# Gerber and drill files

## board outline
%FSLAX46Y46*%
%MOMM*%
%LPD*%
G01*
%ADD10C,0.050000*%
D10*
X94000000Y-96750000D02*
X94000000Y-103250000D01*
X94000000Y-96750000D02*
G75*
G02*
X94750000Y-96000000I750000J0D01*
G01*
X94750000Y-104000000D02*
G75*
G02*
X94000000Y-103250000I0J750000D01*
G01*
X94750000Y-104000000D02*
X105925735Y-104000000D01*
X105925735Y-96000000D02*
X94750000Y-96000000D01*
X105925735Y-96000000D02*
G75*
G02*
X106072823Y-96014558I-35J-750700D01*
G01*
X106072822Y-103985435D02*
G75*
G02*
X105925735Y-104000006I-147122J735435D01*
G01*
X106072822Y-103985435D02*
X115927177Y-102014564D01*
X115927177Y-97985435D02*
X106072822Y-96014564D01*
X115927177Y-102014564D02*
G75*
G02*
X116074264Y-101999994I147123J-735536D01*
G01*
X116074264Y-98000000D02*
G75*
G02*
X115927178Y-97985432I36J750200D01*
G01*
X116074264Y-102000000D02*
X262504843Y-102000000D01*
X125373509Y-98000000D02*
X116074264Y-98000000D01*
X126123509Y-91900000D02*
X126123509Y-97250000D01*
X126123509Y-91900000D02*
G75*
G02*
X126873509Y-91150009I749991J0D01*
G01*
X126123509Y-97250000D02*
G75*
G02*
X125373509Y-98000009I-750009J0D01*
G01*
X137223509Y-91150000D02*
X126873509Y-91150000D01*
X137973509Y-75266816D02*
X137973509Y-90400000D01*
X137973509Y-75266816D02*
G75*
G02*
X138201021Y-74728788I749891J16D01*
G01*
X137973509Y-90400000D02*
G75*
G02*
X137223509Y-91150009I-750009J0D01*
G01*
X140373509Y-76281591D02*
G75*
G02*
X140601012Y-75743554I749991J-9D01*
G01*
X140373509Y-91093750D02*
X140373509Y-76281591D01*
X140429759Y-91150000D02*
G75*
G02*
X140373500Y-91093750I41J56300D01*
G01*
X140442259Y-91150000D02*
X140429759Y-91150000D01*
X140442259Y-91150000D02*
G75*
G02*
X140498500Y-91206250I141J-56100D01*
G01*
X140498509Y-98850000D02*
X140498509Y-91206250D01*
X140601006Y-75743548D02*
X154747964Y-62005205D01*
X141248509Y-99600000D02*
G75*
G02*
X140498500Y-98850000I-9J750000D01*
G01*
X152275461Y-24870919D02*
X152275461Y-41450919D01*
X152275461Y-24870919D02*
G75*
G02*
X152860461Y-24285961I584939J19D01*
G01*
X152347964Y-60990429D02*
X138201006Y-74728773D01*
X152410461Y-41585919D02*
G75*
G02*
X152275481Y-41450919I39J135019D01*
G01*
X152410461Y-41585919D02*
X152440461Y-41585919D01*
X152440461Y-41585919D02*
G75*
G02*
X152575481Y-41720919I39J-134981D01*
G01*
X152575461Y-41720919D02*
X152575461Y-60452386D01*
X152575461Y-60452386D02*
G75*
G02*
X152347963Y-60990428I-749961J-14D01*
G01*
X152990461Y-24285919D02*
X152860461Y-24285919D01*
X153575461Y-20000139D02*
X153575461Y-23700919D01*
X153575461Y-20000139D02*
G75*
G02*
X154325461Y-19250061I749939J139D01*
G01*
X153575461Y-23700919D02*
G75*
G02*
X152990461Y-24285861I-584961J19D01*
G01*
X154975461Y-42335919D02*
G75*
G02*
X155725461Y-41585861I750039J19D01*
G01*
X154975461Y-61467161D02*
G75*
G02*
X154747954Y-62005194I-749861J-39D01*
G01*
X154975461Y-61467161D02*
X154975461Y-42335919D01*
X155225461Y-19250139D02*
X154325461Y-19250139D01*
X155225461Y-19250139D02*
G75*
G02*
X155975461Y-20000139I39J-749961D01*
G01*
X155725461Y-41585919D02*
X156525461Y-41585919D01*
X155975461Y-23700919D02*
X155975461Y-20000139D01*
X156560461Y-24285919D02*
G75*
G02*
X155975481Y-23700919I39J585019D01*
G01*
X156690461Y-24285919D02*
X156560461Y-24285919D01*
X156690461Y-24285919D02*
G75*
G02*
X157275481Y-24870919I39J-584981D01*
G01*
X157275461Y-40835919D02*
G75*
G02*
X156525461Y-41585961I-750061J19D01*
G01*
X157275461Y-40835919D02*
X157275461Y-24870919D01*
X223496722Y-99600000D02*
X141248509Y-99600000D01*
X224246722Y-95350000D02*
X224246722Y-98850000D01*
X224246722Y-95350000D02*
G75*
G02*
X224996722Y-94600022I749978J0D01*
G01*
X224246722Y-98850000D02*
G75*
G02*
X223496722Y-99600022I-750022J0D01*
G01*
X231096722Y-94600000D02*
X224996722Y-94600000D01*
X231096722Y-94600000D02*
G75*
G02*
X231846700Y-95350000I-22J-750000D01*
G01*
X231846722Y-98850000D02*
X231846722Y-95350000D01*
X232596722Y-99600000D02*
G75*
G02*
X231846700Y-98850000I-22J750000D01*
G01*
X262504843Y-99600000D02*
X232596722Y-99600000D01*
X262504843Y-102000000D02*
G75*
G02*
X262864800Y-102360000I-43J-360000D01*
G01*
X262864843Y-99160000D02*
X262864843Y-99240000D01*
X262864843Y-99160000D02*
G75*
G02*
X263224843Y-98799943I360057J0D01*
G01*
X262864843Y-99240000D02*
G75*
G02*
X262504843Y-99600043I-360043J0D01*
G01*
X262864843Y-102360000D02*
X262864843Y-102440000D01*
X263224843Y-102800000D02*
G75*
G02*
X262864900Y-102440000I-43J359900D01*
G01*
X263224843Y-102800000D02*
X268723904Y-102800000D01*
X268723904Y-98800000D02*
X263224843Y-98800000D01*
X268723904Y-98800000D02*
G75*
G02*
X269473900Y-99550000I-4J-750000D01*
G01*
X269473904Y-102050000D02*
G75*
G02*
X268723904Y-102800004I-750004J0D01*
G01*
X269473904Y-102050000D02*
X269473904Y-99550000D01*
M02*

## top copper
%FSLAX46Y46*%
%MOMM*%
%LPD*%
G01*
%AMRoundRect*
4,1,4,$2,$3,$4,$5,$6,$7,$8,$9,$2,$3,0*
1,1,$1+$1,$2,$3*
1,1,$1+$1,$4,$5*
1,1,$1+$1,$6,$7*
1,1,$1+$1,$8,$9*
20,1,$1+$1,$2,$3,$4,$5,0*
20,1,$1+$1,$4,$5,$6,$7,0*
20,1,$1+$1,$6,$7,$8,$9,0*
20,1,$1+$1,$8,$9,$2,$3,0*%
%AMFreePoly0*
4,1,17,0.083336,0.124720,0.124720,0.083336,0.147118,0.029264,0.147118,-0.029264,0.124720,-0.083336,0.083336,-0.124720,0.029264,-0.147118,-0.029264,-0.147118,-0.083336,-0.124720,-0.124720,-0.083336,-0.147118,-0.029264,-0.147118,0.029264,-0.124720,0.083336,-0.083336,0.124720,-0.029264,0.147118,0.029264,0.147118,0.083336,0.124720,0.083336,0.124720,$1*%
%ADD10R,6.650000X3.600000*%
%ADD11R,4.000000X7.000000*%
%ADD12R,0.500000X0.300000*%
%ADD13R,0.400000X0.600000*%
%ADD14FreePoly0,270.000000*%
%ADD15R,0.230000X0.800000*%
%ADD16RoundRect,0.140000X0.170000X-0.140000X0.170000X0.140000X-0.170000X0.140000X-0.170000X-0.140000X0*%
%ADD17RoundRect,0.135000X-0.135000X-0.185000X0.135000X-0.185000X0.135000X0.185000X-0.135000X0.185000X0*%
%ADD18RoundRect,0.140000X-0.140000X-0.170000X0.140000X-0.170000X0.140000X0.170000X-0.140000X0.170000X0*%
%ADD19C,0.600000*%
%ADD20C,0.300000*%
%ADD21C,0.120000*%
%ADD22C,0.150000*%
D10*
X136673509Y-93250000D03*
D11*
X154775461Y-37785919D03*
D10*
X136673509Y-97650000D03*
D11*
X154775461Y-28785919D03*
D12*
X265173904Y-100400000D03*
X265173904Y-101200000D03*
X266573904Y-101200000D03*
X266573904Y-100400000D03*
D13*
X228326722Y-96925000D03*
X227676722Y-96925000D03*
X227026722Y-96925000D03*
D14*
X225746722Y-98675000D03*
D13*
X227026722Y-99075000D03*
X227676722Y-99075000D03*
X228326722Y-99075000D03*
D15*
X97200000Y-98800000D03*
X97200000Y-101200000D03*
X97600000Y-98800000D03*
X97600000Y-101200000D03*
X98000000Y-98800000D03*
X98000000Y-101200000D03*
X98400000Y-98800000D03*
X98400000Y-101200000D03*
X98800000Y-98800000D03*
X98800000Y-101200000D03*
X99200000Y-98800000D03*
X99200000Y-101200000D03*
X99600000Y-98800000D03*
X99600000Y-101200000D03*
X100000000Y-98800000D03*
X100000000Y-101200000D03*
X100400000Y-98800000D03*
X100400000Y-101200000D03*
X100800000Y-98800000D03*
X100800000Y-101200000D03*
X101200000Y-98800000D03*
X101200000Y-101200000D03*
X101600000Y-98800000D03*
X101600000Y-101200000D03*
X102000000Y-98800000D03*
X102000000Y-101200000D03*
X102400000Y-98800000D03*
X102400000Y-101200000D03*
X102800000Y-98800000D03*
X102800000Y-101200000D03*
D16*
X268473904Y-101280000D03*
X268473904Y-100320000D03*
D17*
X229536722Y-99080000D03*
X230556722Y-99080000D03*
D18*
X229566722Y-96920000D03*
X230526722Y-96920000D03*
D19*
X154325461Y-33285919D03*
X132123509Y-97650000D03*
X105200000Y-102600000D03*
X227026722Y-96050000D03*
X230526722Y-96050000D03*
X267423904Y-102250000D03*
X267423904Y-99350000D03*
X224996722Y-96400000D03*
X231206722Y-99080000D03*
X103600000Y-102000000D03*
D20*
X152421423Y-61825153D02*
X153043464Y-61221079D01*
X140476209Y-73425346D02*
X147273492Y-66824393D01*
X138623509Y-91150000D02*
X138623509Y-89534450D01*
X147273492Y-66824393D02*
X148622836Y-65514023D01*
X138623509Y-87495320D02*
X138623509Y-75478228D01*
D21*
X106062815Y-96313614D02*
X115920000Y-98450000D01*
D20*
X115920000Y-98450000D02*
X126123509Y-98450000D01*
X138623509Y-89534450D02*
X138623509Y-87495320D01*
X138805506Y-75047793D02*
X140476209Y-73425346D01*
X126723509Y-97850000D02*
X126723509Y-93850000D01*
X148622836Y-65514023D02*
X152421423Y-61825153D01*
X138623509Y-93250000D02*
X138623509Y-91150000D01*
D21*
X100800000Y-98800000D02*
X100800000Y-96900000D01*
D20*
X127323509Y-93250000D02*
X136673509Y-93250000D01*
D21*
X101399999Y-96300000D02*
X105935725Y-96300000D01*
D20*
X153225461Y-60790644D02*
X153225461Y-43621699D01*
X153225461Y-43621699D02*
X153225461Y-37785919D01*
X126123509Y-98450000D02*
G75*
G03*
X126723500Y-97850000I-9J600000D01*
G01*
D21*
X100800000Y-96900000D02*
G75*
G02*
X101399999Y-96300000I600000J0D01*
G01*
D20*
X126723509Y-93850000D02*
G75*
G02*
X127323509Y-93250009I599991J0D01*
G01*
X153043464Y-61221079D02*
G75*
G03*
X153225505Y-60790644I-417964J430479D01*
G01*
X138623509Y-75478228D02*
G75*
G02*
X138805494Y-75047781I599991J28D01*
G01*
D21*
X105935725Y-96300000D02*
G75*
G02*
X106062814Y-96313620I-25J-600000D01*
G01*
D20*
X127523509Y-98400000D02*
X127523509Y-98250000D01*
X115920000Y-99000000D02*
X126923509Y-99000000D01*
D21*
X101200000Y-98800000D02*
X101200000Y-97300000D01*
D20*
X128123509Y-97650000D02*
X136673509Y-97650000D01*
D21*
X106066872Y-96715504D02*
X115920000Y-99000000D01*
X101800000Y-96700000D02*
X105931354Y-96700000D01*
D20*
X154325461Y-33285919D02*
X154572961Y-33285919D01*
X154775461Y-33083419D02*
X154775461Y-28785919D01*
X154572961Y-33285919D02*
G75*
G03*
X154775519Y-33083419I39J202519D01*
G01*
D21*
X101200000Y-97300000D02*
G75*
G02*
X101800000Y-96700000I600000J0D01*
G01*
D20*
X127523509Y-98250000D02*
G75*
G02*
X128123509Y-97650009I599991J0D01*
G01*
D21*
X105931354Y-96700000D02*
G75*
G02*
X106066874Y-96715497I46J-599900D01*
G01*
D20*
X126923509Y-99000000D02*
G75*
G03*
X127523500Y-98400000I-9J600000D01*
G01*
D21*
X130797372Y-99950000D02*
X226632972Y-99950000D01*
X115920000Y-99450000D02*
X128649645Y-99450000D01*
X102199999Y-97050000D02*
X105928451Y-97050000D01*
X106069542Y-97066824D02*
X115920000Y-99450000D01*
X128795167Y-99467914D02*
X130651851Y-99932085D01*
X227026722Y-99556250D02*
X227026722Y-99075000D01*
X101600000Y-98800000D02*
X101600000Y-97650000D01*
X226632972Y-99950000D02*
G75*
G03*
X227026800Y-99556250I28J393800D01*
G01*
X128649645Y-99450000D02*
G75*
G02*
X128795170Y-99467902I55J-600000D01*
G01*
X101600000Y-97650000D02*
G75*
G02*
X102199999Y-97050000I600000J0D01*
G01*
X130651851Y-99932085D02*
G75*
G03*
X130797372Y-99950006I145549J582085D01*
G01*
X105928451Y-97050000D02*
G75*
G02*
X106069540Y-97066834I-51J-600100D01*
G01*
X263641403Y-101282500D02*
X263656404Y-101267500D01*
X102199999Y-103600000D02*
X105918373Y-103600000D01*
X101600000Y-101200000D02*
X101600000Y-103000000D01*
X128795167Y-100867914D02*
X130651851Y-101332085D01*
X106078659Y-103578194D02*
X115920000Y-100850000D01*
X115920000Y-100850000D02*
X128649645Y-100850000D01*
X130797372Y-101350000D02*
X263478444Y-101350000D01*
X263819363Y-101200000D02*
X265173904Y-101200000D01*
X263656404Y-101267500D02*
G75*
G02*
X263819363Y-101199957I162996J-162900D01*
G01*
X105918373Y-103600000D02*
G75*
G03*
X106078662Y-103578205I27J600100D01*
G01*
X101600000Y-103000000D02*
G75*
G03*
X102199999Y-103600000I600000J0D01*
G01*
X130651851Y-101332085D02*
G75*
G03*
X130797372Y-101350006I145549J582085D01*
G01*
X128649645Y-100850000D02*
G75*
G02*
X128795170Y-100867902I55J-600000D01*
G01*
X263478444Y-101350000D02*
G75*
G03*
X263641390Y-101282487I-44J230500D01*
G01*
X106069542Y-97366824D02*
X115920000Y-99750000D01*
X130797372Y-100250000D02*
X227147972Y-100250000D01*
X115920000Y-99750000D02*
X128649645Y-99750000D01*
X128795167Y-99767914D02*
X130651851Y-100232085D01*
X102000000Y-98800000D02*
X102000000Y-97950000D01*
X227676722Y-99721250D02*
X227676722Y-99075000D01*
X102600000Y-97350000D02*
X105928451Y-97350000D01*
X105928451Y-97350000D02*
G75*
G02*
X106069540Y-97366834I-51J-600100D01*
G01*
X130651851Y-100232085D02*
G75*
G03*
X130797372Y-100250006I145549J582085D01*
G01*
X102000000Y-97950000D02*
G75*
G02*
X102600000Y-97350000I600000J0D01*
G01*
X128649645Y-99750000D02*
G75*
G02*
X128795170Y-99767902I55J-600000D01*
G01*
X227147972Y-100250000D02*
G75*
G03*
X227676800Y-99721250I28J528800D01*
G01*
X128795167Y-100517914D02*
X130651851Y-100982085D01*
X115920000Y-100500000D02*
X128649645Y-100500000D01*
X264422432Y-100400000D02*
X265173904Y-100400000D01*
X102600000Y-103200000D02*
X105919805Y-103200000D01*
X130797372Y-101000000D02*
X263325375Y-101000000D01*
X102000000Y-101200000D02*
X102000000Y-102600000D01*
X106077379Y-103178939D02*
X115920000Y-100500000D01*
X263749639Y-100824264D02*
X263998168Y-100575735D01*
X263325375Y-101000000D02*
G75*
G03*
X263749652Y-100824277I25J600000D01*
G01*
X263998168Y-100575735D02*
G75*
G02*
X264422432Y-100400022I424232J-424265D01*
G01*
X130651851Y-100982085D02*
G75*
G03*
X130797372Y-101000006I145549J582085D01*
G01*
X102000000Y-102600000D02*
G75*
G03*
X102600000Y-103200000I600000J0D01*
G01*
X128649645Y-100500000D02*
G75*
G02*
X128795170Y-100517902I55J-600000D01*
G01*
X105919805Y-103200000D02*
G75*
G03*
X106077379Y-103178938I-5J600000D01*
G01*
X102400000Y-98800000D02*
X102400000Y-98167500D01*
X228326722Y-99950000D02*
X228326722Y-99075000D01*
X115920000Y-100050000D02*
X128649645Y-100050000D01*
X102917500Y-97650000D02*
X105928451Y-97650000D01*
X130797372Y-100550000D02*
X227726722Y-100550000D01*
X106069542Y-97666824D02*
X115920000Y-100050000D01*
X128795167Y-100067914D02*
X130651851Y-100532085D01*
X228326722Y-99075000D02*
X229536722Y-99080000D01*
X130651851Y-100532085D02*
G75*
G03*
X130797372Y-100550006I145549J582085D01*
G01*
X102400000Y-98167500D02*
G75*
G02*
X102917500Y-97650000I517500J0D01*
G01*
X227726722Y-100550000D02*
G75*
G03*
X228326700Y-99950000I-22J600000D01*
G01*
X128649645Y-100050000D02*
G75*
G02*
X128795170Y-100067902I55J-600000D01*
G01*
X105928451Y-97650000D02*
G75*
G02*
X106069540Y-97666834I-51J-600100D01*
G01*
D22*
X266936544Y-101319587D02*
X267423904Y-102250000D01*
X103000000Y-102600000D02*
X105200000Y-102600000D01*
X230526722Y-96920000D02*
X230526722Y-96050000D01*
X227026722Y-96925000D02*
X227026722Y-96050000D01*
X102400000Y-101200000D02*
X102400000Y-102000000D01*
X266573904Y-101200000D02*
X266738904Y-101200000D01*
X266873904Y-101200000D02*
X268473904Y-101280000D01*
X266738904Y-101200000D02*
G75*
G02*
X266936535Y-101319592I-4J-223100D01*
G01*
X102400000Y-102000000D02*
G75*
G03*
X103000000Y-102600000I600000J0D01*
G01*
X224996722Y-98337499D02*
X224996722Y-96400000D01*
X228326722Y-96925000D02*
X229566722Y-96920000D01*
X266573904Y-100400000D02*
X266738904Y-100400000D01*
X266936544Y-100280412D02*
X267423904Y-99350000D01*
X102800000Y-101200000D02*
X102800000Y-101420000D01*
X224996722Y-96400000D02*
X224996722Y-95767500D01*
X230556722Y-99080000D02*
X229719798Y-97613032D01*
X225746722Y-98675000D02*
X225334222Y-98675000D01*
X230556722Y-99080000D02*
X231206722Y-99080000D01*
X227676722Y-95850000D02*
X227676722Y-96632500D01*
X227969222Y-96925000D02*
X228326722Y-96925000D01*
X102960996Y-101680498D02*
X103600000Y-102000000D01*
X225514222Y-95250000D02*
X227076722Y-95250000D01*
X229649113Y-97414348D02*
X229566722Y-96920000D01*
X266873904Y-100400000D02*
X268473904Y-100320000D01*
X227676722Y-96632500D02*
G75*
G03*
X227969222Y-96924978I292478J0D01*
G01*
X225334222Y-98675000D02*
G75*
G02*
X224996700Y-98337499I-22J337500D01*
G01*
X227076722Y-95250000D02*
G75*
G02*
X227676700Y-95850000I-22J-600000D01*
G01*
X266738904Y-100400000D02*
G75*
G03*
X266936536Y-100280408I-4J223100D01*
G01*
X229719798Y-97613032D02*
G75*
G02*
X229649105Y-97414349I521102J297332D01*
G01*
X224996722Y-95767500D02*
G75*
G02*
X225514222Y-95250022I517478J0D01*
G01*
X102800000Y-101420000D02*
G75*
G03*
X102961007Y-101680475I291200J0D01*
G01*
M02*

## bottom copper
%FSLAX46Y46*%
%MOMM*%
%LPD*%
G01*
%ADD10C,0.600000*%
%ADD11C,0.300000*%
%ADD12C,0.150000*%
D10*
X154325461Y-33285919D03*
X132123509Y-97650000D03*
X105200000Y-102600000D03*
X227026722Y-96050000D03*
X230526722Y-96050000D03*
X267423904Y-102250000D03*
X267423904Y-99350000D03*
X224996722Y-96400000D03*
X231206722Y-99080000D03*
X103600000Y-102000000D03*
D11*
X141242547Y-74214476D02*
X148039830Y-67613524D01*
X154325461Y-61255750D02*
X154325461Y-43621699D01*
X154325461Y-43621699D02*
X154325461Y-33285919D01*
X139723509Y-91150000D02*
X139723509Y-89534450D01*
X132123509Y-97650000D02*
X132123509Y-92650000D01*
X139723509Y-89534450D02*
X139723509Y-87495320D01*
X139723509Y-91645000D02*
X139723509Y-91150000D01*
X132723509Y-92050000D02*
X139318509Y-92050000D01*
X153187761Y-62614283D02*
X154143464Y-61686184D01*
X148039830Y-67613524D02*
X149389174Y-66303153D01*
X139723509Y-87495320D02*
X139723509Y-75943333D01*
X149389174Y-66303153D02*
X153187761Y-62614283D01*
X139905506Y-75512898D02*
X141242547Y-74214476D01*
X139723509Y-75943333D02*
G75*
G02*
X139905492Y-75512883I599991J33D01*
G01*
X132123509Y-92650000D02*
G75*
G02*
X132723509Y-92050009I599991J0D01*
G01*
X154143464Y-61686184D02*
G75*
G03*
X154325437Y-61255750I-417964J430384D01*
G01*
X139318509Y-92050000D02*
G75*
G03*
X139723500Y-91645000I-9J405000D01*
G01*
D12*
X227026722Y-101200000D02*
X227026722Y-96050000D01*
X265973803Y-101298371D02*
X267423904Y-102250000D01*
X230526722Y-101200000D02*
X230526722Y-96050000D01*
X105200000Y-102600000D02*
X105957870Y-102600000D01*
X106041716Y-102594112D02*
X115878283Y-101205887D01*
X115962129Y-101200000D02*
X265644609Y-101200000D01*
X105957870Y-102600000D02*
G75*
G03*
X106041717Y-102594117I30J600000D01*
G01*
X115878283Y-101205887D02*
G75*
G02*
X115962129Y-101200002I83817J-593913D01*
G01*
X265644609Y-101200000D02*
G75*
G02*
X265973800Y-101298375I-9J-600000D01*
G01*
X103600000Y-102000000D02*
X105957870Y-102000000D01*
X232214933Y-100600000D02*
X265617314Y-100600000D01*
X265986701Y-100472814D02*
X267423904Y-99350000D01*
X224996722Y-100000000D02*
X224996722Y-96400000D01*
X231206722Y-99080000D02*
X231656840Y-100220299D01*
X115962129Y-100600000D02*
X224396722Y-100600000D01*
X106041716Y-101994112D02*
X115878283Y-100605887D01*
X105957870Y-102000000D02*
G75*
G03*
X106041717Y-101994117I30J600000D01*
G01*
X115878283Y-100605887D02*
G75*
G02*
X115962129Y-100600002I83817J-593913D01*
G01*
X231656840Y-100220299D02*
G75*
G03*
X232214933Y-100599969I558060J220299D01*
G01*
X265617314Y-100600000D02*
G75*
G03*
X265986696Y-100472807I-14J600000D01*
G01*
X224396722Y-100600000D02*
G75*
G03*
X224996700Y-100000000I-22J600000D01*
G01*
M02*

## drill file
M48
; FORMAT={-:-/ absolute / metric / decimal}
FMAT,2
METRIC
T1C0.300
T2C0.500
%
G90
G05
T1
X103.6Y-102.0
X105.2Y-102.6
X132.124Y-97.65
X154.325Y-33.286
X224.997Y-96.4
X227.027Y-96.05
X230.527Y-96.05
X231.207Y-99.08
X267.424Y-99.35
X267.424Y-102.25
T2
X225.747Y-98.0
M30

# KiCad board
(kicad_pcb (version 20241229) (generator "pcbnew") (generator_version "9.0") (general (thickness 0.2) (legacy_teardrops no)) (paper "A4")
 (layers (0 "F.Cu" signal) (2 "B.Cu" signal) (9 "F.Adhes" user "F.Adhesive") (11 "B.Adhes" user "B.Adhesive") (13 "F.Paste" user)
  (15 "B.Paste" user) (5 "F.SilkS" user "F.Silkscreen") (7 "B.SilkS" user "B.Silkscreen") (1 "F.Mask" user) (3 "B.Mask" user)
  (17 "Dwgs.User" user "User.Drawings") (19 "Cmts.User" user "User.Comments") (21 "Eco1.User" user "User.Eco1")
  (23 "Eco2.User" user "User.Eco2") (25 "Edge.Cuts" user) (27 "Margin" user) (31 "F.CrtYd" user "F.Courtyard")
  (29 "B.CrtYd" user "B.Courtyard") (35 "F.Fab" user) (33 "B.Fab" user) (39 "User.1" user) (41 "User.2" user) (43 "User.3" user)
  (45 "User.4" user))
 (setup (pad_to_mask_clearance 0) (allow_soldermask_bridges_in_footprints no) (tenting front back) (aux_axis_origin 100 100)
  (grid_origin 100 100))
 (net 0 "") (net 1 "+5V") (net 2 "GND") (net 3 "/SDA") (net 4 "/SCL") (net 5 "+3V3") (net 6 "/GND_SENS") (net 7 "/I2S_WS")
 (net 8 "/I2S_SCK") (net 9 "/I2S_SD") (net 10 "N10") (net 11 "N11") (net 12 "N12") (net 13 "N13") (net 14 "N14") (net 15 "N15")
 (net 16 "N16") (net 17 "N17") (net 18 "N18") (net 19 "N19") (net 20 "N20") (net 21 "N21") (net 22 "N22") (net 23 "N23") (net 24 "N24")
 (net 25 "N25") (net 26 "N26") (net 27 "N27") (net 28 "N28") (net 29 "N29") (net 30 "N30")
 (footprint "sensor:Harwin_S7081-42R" (layer "F.Cu") (at 136.673509 93.25)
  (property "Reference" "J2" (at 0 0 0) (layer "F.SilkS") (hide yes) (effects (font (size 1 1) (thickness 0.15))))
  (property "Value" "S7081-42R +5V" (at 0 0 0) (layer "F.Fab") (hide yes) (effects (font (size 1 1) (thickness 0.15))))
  (pad "1" smd rect (at 0 0) (size 6.65 3.6) (layers "F.Cu" "F.Mask" "F.Paste") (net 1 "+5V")))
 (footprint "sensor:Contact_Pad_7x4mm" (layer "F.Cu") (at 154.775461 37.785919 90)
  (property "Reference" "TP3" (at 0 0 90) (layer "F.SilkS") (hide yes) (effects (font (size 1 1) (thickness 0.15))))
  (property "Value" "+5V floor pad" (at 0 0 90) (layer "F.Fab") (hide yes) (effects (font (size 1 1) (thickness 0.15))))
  (pad "1" smd rect (at 0 0 90) (size 7 4) (layers "F.Cu" "F.Mask") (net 1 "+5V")))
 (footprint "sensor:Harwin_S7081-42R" (layer "F.Cu") (at 136.673509 97.65)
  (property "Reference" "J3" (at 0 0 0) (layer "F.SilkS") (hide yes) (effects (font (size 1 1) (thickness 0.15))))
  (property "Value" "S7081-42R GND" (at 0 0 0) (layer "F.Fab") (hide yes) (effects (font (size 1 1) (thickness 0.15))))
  (pad "1" smd rect (at 0 0) (size 6.65 3.6) (layers "F.Cu" "F.Mask" "F.Paste") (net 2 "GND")))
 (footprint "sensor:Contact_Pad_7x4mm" (layer "F.Cu") (at 154.775461 28.785919 90)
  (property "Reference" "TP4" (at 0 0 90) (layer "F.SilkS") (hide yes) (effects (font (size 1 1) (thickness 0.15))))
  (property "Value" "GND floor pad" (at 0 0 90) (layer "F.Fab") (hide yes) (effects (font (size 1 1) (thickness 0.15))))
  (pad "1" smd rect (at 0 0 90) (size 7 4) (layers "F.Cu" "F.Mask") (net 2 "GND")))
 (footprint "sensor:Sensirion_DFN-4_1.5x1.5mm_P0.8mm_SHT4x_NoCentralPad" (layer "F.Cu") (at 265.873904 100.8)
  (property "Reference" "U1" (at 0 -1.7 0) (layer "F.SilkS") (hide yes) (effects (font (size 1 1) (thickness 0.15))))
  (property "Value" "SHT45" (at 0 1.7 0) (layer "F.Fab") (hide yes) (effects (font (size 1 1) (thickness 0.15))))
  (pad "1" smd rect (at -0.7 -0.4) (size 0.5 0.3) (layers "F.Cu" "F.Mask" "F.Paste") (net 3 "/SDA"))
  (pad "2" smd rect (at -0.7 0.4) (size 0.5 0.3) (layers "F.Cu" "F.Mask" "F.Paste") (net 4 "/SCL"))
  (pad "3" smd rect (at 0.7 0.4) (size 0.5 0.3) (layers "F.Cu" "F.Mask" "F.Paste") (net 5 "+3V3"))
  (pad "4" smd rect (at 0.7 -0.4) (size 0.5 0.3) (layers "F.Cu" "F.Mask" "F.Paste") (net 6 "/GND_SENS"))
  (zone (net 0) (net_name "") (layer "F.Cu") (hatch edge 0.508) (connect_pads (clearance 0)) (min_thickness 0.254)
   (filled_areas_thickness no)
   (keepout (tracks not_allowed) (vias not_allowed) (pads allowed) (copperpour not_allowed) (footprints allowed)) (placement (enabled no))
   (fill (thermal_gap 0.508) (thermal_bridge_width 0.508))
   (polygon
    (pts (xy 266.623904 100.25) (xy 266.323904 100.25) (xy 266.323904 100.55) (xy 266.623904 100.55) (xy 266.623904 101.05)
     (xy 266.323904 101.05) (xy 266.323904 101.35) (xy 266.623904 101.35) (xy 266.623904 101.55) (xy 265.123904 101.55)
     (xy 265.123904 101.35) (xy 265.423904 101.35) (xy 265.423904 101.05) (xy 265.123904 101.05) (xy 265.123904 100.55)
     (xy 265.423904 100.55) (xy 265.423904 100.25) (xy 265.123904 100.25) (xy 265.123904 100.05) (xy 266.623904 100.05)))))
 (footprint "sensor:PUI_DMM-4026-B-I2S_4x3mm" (layer "F.Cu") (at 226.746722 98 -90)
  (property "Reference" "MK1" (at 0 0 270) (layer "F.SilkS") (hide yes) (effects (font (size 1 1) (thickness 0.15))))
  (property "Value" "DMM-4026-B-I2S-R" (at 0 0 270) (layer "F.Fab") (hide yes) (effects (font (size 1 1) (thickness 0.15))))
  (pad "" np_thru_hole circle (at 0 1 270) (size 0.5 0.5) (drill 0.5) (layers "*.Mask"))
  (pad "1" smd rect (at -1.075 -1.58 270) (size 0.6 0.4) (layers "F.Cu" "F.Mask" "F.Paste") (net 6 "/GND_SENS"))
  (pad "2" smd rect (at -1.075 -0.93 270) (size 0.6 0.4) (layers "F.Cu" "F.Mask" "F.Paste") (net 6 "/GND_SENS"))
  (pad "3" smd rect (at -1.075 -0.28 270) (size 0.6 0.4) (layers "F.Cu" "F.Mask" "F.Paste") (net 5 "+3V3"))
  (pad "4" smd custom (at 0.675 1 270) (size 0.3 0.3) (layers "F.Cu" "F.Mask" "F.Paste") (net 6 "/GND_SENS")
   (options (clearance outline) (anchor circle)) (primitives))
  (pad "5" smd rect (at 1.075 -0.28 270) (size 0.6 0.4) (layers "F.Cu" "F.Mask" "F.Paste") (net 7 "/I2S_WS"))
  (pad "6" smd rect (at 1.075 -0.93 270) (size 0.6 0.4) (layers "F.Cu" "F.Mask" "F.Paste") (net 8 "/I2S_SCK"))
  (pad "7" smd rect (at 1.075 -1.58 270) (size 0.6 0.4) (layers "F.Cu" "F.Mask" "F.Paste") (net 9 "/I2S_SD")))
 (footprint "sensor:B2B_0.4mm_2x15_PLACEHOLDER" (layer "F.Cu") (at 100 100)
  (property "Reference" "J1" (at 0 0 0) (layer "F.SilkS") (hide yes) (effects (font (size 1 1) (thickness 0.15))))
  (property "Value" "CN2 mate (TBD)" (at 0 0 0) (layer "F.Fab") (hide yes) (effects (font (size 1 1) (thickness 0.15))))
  (pad "1" smd rect (at -2.8 -1.2) (size 0.23 0.8) (layers "F.Cu" "F.Mask" "F.Paste") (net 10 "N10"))
  (pad "2" smd rect (at -2.8 1.2) (size 0.23 0.8) (layers "F.Cu" "F.Mask" "F.Paste") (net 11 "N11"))
  (pad "3" smd rect (at -2.4 -1.2) (size 0.23 0.8) (layers "F.Cu" "F.Mask" "F.Paste") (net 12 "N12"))
  (pad "4" smd rect (at -2.4 1.2) (size 0.23 0.8) (layers "F.Cu" "F.Mask" "F.Paste") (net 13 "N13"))
  (pad "5" smd rect (at -2 -1.2) (size 0.23 0.8) (layers "F.Cu" "F.Mask" "F.Paste") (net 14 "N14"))
  (pad "6" smd rect (at -2 1.2) (size 0.23 0.8) (layers "F.Cu" "F.Mask" "F.Paste") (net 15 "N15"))
  (pad "7" smd rect (at -1.6 -1.2) (size 0.23 0.8) (layers "F.Cu" "F.Mask" "F.Paste") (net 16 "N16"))
  (pad "8" smd rect (at -1.6 1.2) (size 0.23 0.8) (layers "F.Cu" "F.Mask" "F.Paste") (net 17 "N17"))
  (pad "9" smd rect (at -1.2 -1.2) (size 0.23 0.8) (layers "F.Cu" "F.Mask" "F.Paste") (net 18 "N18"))
  (pad "10" smd rect (at -1.2 1.2) (size 0.23 0.8) (layers "F.Cu" "F.Mask" "F.Paste") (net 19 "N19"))
  (pad "11" smd rect (at -0.8 -1.2) (size 0.23 0.8) (layers "F.Cu" "F.Mask" "F.Paste") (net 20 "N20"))
  (pad "12" smd rect (at -0.8 1.2) (size 0.23 0.8) (layers "F.Cu" "F.Mask" "F.Paste") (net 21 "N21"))
  (pad "13" smd rect (at -0.4 -1.2) (size 0.23 0.8) (layers "F.Cu" "F.Mask" "F.Paste") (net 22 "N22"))
  (pad "14" smd rect (at -0.4 1.2) (size 0.23 0.8) (layers "F.Cu" "F.Mask" "F.Paste") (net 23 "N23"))
  (pad "15" smd rect (at 0 -1.2) (size 0.23 0.8) (layers "F.Cu" "F.Mask" "F.Paste") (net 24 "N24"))
  (pad "16" smd rect (at 0 1.2) (size 0.23 0.8) (layers "F.Cu" "F.Mask" "F.Paste") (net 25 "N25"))
  (pad "17" smd rect (at 0.4 -1.2) (size 0.23 0.8) (layers "F.Cu" "F.Mask" "F.Paste") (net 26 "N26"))
  (pad "18" smd rect (at 0.4 1.2) (size 0.23 0.8) (layers "F.Cu" "F.Mask" "F.Paste") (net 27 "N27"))
  (pad "19" smd rect (at 0.8 -1.2) (size 0.23 0.8) (layers "F.Cu" "F.Mask" "F.Paste") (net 1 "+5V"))
  (pad "20" smd rect (at 0.8 1.2) (size 0.23 0.8) (layers "F.Cu" "F.Mask" "F.Paste") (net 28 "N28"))
  (pad "21" smd rect (at 1.2 -1.2) (size 0.23 0.8) (layers "F.Cu" "F.Mask" "F.Paste") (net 2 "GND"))
  (pad "22" smd rect (at 1.2 1.2) (size 0.23 0.8) (layers "F.Cu" "F.Mask" "F.Paste") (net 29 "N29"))
  (pad "23" smd rect (at 1.6 -1.2) (size 0.23 0.8) (layers "F.Cu" "F.Mask" "F.Paste") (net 7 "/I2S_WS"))
  (pad "24" smd rect (at 1.6 1.2) (size 0.23 0.8) (layers "F.Cu" "F.Mask" "F.Paste") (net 4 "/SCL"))
  (pad "25" smd rect (at 2 -1.2) (size 0.23 0.8) (layers "F.Cu" "F.Mask" "F.Paste") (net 8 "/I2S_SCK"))
  (pad "26" smd rect (at 2 1.2) (size 0.23 0.8) (layers "F.Cu" "F.Mask" "F.Paste") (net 3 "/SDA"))
  (pad "27" smd rect (at 2.4 -1.2) (size 0.23 0.8) (layers "F.Cu" "F.Mask" "F.Paste") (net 9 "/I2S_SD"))
  (pad "28" smd rect (at 2.4 1.2) (size 0.23 0.8) (layers "F.Cu" "F.Mask" "F.Paste") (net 5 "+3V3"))
  (pad "29" smd rect (at 2.8 -1.2) (size 0.23 0.8) (layers "F.Cu" "F.Mask" "F.Paste") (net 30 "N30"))
  (pad "30" smd rect (at 2.8 1.2) (size 0.23 0.8) (layers "F.Cu" "F.Mask" "F.Paste") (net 6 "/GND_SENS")))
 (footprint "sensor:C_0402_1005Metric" (layer "F.Cu") (at 268.473904 100.8 90)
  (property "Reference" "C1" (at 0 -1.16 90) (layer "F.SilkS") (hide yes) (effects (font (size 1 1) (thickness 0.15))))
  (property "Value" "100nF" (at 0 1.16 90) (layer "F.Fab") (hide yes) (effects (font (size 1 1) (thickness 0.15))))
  (pad "1" smd roundrect (at -0.48 0 90) (size 0.56 0.62) (layers "F.Cu" "F.Mask" "F.Paste") (roundrect_rratio 0.25) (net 5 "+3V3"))
  (pad "2" smd roundrect (at 0.48 0 90) (size 0.56 0.62) (layers "F.Cu" "F.Mask" "F.Paste") (roundrect_rratio 0.25) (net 6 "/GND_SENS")))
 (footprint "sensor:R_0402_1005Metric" (layer "F.Cu") (at 230.046722 99.08)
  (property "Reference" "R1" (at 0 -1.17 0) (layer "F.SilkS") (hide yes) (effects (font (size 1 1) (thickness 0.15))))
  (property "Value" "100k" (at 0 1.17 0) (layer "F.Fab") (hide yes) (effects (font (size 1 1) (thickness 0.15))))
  (pad "1" smd roundrect (at -0.51 0) (size 0.54 0.64) (layers "F.Cu" "F.Mask" "F.Paste") (roundrect_rratio 0.25) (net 9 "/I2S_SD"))
  (pad "2" smd roundrect (at 0.51 0) (size 0.54 0.64) (layers "F.Cu" "F.Mask" "F.Paste") (roundrect_rratio 0.25) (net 6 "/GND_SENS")))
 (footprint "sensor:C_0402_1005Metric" (layer "F.Cu") (at 230.046722 96.92)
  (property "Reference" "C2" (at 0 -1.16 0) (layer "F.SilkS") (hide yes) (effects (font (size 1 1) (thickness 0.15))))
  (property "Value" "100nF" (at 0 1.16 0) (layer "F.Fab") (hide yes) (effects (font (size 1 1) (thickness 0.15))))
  (pad "1" smd roundrect (at -0.48 0) (size 0.56 0.62) (layers "F.Cu" "F.Mask" "F.Paste") (roundrect_rratio 0.25) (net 6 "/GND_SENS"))
  (pad "2" smd roundrect (at 0.48 0) (size 0.56 0.62) (layers "F.Cu" "F.Mask" "F.Paste") (roundrect_rratio 0.25) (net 5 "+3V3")))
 (gr_line (start 94 96.75) (end 94 103.25) (stroke (width 0.05) (type default)) (layer "Edge.Cuts"))
 (gr_arc (start 94 96.75) (mid 94.21967 96.21967) (end 94.75 96) (stroke (width 0.05) (type default)) (layer "Edge.Cuts"))
 (gr_arc (start 94.75 104) (mid 94.21967 103.78033) (end 94 103.25) (stroke (width 0.05) (type default)) (layer "Edge.Cuts"))
 (gr_line (start 94.75 104) (end 105.925735 104) (stroke (width 0.05) (type default)) (layer "Edge.Cuts"))
 (gr_line (start 105.925735 96) (end 94.75 96) (stroke (width 0.05) (type default)) (layer "Edge.Cuts"))
 (gr_arc (start 105.925735 96) (mid 105.999638 96.003653) (end 106.072822 96.014564) (stroke (width 0.05) (type default))
  (layer "Edge.Cuts"))
 (gr_arc (start 106.072822 103.985435) (mid 105.999638 103.99635) (end 105.925735 104) (stroke (width 0.05) (type default))
  (layer "Edge.Cuts"))
 (gr_line (start 106.072822 103.985435) (end 115.927177 102.014564) (stroke (width 0.05) (type default)) (layer "Edge.Cuts"))
 (gr_line (start 115.927177 97.985435) (end 106.072822 96.014564) (stroke (width 0.05) (type default)) (layer "Edge.Cuts"))
 (gr_arc (start 115.927177 102.014564) (mid 116.000361 102.00365) (end 116.074264 102) (stroke (width 0.05) (type default))
  (layer "Edge.Cuts"))
 (gr_arc (start 116.074264 98) (mid 116.000361 97.996349) (end 115.927177 97.985435) (stroke (width 0.05) (type default))
  (layer "Edge.Cuts"))
 (gr_line (start 116.074264 102) (end 262.504843 102) (stroke (width 0.05) (type default)) (layer "Edge.Cuts"))
 (gr_line (start 125.373509 98) (end 116.074264 98) (stroke (width 0.05) (type default)) (layer "Edge.Cuts"))
 (gr_line (start 126.123509 91.9) (end 126.123509 97.25) (stroke (width 0.05) (type default)) (layer "Edge.Cuts"))
 (gr_arc (start 126.123509 91.9) (mid 126.343179 91.369673) (end 126.873509 91.15) (stroke (width 0.05) (type default)) (layer "Edge.Cuts"))
 (gr_arc (start 126.123509 97.25) (mid 125.903839 97.78033) (end 125.373509 98) (stroke (width 0.05) (type default)) (layer "Edge.Cuts"))
 (gr_line (start 137.223509 91.15) (end 126.873509 91.15) (stroke (width 0.05) (type default)) (layer "Edge.Cuts"))
 (gr_line (start 137.973509 75.266816) (end 137.973509 90.4) (stroke (width 0.05) (type default)) (layer "Edge.Cuts"))
 (gr_arc (start 137.973509 75.266816) (mid 138.032716 74.974732) (end 138.201006 74.728773) (stroke (width 0.05) (type default))
  (layer "Edge.Cuts"))
 (gr_arc (start 137.973509 90.4) (mid 137.753839 90.93033) (end 137.223509 91.15) (stroke (width 0.05) (type default)) (layer "Edge.Cuts"))
 (gr_arc (start 140.373509 76.281591) (mid 140.43272 75.98951) (end 140.601006 75.743548) (stroke (width 0.05) (type default))
  (layer "Edge.Cuts"))
 (gr_line (start 140.373509 91.09375) (end 140.373509 76.281591) (stroke (width 0.05) (type default)) (layer "Edge.Cuts"))
 (gr_arc (start 140.429759 91.15) (mid 140.389984 91.133524) (end 140.373509 91.09375) (stroke (width 0.05) (type default))
  (layer "Edge.Cuts"))
 (gr_line (start 140.442259 91.15) (end 140.429759 91.15) (stroke (width 0.05) (type default)) (layer "Edge.Cuts"))
 (gr_arc (start 140.442259 91.15) (mid 140.482078 91.166458) (end 140.498509 91.20625) (stroke (width 0.05) (type default))
  (layer "Edge.Cuts"))
 (gr_line (start 140.498509 98.85) (end 140.498509 91.20625) (stroke (width 0.05) (type default)) (layer "Edge.Cuts"))
 (gr_line (start 140.601006 75.743548) (end 154.747964 62.005205) (stroke (width 0.05) (type default)) (layer "Edge.Cuts"))
 (gr_arc (start 141.248509 99.6) (mid 140.718179 99.38033) (end 140.498509 98.85) (stroke (width 0.05) (type default)) (layer "Edge.Cuts"))
 (gr_line (start 152.275461 24.870919) (end 152.275461 41.450919) (stroke (width 0.05) (type default)) (layer "Edge.Cuts"))
 (gr_arc (start 152.275461 24.870919) (mid 152.446794 24.457235) (end 152.860461 24.285919) (stroke (width 0.05) (type default))
  (layer "Edge.Cuts"))
 (gr_line (start 152.347964 60.990429) (end 138.201006 74.728773) (stroke (width 0.05) (type default)) (layer "Edge.Cuts"))
 (gr_arc (start 152.410461 41.585919) (mid 152.31502 41.546366) (end 152.275461 41.450919) (stroke (width 0.05) (type default))
  (layer "Edge.Cuts"))
 (gr_line (start 152.410461 41.585919) (end 152.440461 41.585919) (stroke (width 0.05) (type default)) (layer "Edge.Cuts"))
 (gr_arc (start 152.440461 41.585919) (mid 152.535921 41.625459) (end 152.575461 41.720919) (stroke (width 0.05) (type default))
  (layer "Edge.Cuts"))
 (gr_line (start 152.575461 41.720919) (end 152.575461 60.452386) (stroke (width 0.05) (type default)) (layer "Edge.Cuts"))
 (gr_arc (start 152.575461 60.452386) (mid 152.51625 60.744467) (end 152.347964 60.990429) (stroke (width 0.05) (type default))
  (layer "Edge.Cuts"))
 (gr_line (start 152.990461 24.285919) (end 152.860461 24.285919) (stroke (width 0.05) (type default)) (layer "Edge.Cuts"))
 (gr_line (start 153.575461 20.000139) (end 153.575461 23.700919) (stroke (width 0.05) (type default)) (layer "Edge.Cuts"))
 (gr_arc (start 153.575461 20.000139) (mid 153.795115 19.46977) (end 154.325461 19.250139) (stroke (width 0.05) (type default))
  (layer "Edge.Cuts"))
 (gr_arc (start 153.575461 23.700919) (mid 153.404119 24.114576) (end 152.990461 24.285919) (stroke (width 0.05) (type default))
  (layer "Edge.Cuts"))
 (gr_arc (start 154.975461 42.335919) (mid 155.195131 41.805588) (end 155.725461 41.585919) (stroke (width 0.05) (type default))
  (layer "Edge.Cuts"))
 (gr_arc (start 154.975461 61.467161) (mid 154.91626 61.759249) (end 154.747964 62.005205) (stroke (width 0.05) (type default))
  (layer "Edge.Cuts"))
 (gr_line (start 154.975461 61.467161) (end 154.975461 42.335919) (stroke (width 0.05) (type default)) (layer "Edge.Cuts"))
 (gr_line (start 155.225461 19.250139) (end 154.325461 19.250139) (stroke (width 0.05) (type default)) (layer "Edge.Cuts"))
 (gr_arc (start 155.225461 19.250139) (mid 155.755803 19.469797) (end 155.975461 20.000139) (stroke (width 0.05) (type default))
  (layer "Edge.Cuts"))
 (gr_line (start 155.725461 41.585919) (end 156.525461 41.585919) (stroke (width 0.05) (type default)) (layer "Edge.Cuts"))
 (gr_line (start 155.975461 23.700919) (end 155.975461 20.000139) (stroke (width 0.05) (type default)) (layer "Edge.Cuts"))
 (gr_arc (start 156.560461 24.285919) (mid 156.146804 24.114576) (end 155.975461 23.700919) (stroke (width 0.05) (type default))
  (layer "Edge.Cuts"))
 (gr_line (start 156.690461 24.285919) (end 156.560461 24.285919) (stroke (width 0.05) (type default)) (layer "Edge.Cuts"))
 (gr_arc (start 156.690461 24.285919) (mid 157.104137 24.457249) (end 157.275461 24.870919) (stroke (width 0.05) (type default))
  (layer "Edge.Cuts"))
 (gr_arc (start 157.275461 40.835919) (mid 157.055782 41.366223) (end 156.525461 41.585919) (stroke (width 0.05) (type default))
  (layer "Edge.Cuts"))
 (gr_line (start 157.275461 40.835919) (end 157.275461 24.870919) (stroke (width 0.05) (type default)) (layer "Edge.Cuts"))
 (gr_line (start 223.496722 99.6) (end 141.248509 99.6) (stroke (width 0.05) (type default)) (layer "Edge.Cuts"))
 (gr_line (start 224.246722 95.35) (end 224.246722 98.85) (stroke (width 0.05) (type default)) (layer "Edge.Cuts"))
 (gr_arc (start 224.246722 95.35) (mid 224.466393 94.819678) (end 224.996722 94.6) (stroke (width 0.05) (type default)) (layer "Edge.Cuts"))
 (gr_arc (start 224.246722 98.85) (mid 224.027052 99.38033) (end 223.496722 99.6) (stroke (width 0.05) (type default)) (layer "Edge.Cuts"))
 (gr_line (start 231.096722 94.6) (end 224.996722 94.6) (stroke (width 0.05) (type default)) (layer "Edge.Cuts"))
 (gr_arc (start 231.096722 94.6) (mid 231.627038 94.819678) (end 231.846722 95.35) (stroke (width 0.05) (type default)) (layer "Edge.Cuts"))
 (gr_line (start 231.846722 98.85) (end 231.846722 95.35) (stroke (width 0.05) (type default)) (layer "Edge.Cuts"))
 (gr_arc (start 232.596722 99.6) (mid 232.066392 99.38033) (end 231.846722 98.85) (stroke (width 0.05) (type default)) (layer "Edge.Cuts"))
 (gr_line (start 262.504843 99.6) (end 232.596722 99.6) (stroke (width 0.05) (type default)) (layer "Edge.Cuts"))
 (gr_arc (start 262.504843 102) (mid 262.759402 102.105441) (end 262.864843 102.36) (stroke (width 0.05) (type default)) (layer "Edge.Cuts"))
 (gr_line (start 262.864843 99.16) (end 262.864843 99.24) (stroke (width 0.05) (type default)) (layer "Edge.Cuts"))
 (gr_arc (start 262.864843 99.16) (mid 262.970287 98.905457) (end 263.224843 98.8) (stroke (width 0.05) (type default)) (layer "Edge.Cuts"))
 (gr_arc (start 262.864843 99.24) (mid 262.759402 99.494558) (end 262.504843 99.6) (stroke (width 0.05) (type default)) (layer "Edge.Cuts"))
 (gr_line (start 262.864843 102.36) (end 262.864843 102.44) (stroke (width 0.05) (type default)) (layer "Edge.Cuts"))
 (gr_arc (start 263.224843 102.8) (mid 262.970257 102.694574) (end 262.864843 102.44) (stroke (width 0.05) (type default))
  (layer "Edge.Cuts"))
 (gr_line (start 263.224843 102.8) (end 268.723904 102.8) (stroke (width 0.05) (type default)) (layer "Edge.Cuts"))
 (gr_line (start 268.723904 98.8) (end 263.224843 98.8) (stroke (width 0.05) (type default)) (layer "Edge.Cuts"))
 (gr_arc (start 268.723904 98.8) (mid 269.254232 99.019671) (end 269.473904 99.55) (stroke (width 0.05) (type default)) (layer "Edge.Cuts"))
 (gr_arc (start 269.473904 102.05) (mid 269.254234 102.580332) (end 268.723904 102.8) (stroke (width 0.05) (type default))
  (layer "Edge.Cuts"))
 (gr_line (start 269.473904 102.05) (end 269.473904 99.55) (stroke (width 0.05) (type default)) (layer "Edge.Cuts"))
 (segment (start 152.421423 61.825153) (end 153.043464 61.221079) (width 0.3) (layer "F.Cu") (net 1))
 (segment (start 140.476209 73.425346) (end 147.273492 66.824393) (width 0.3) (layer "F.Cu") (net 1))
 (segment (start 138.623509 91.15) (end 138.623509 89.53445) (width 0.3) (layer "F.Cu") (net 1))
 (segment (start 147.273492 66.824393) (end 148.622836 65.514023) (width 0.3) (layer "F.Cu") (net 1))
 (segment (start 138.623509 87.49532) (end 138.623509 75.478228) (width 0.3) (layer "F.Cu") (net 1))
 (segment (start 106.062815 96.313614) (end 115.92 98.45) (width 0.12) (layer "F.Cu") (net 1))
 (segment (start 115.92 98.45) (end 126.123509 98.45) (width 0.3) (layer "F.Cu") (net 1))
 (segment (start 138.623509 89.53445) (end 138.623509 87.49532) (width 0.3) (layer "F.Cu") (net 1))
 (segment (start 138.805506 75.047793) (end 140.476209 73.425346) (width 0.3) (layer "F.Cu") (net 1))
 (segment (start 126.723509 97.85) (end 126.723509 93.85) (width 0.3) (layer "F.Cu") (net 1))
 (segment (start 148.622836 65.514023) (end 152.421423 61.825153) (width 0.3) (layer "F.Cu") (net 1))
 (segment (start 138.623509 93.25) (end 138.623509 91.15) (width 0.3) (layer "F.Cu") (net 1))
 (segment (start 100.8 98.8) (end 100.8 96.9) (width 0.12) (layer "F.Cu") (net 1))
 (segment (start 127.323509 93.25) (end 136.673509 93.25) (width 0.3) (layer "F.Cu") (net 1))
 (segment (start 101.399999 96.3) (end 105.935725 96.3) (width 0.12) (layer "F.Cu") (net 1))
 (segment (start 153.225461 60.790644) (end 153.225461 43.621699) (width 0.3) (layer "F.Cu") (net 1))
 (segment (start 153.225461 43.621699) (end 153.225461 37.785919) (width 0.3) (layer "F.Cu") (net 1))
 (arc (start 126.123509 98.45) (mid 126.547773 98.274264) (end 126.723509 97.85) (width 0.3) (layer "F.Cu") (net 1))
 (arc (start 100.8 96.9) (mid 100.975735 96.475735) (end 101.399999 96.3) (width 0.12) (layer "F.Cu") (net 1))
 (arc (start 126.723509 93.85) (mid 126.899245 93.425735) (end 127.323509 93.25) (width 0.3) (layer "F.Cu") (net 1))
 (arc (start 153.043464 61.221079) (mid 153.178092 61.024309) (end 153.225461 60.790644) (width 0.3) (layer "F.Cu") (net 1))
 (arc (start 138.623509 75.478228) (mid 138.670878 75.244563) (end 138.805506 75.047793) (width 0.3) (layer "F.Cu") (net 1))
 (arc (start 105.935725 96.3) (mid 105.999634 96.303413) (end 106.062815 96.313614) (width 0.12) (layer "F.Cu") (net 1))
 (segment (start 127.523509 98.4) (end 127.523509 98.25) (width 0.3) (layer "F.Cu") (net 2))
 (segment (start 115.92 99) (end 126.923509 99) (width 0.3) (layer "F.Cu") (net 2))
 (segment (start 101.2 98.8) (end 101.2 97.3) (width 0.12) (layer "F.Cu") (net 2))
 (segment (start 128.123509 97.65) (end 136.673509 97.65) (width 0.3) (layer "F.Cu") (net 2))
 (segment (start 106.066872 96.715504) (end 115.92 99) (width 0.12) (layer "F.Cu") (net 2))
 (segment (start 101.8 96.7) (end 105.931354 96.7) (width 0.12) (layer "F.Cu") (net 2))
 (segment (start 154.325461 33.285919) (end 154.572961 33.285919) (width 0.3) (layer "F.Cu") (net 2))
 (segment (start 154.775461 33.083419) (end 154.775461 28.785919) (width 0.3) (layer "F.Cu") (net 2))
 (via (at 154.325461 33.285919) (size 0.6) (drill 0.3) (layers "F.Cu" "B.Cu") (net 2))
 (via (at 132.123509 97.65) (size 0.6) (drill 0.3) (layers "F.Cu" "B.Cu") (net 2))
 (arc (start 154.572961 33.285919) (mid 154.71615 33.226608) (end 154.775461 33.083419) (width 0.3) (layer "F.Cu") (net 2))
 (arc (start 101.2 97.3) (mid 101.375735 96.875735) (end 101.8 96.7) (width 0.12) (layer "F.Cu") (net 2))
 (arc (start 127.523509 98.25) (mid 127.699245 97.825735) (end 128.123509 97.65) (width 0.3) (layer "F.Cu") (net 2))
 (arc (start 105.931354 96.7) (mid 105.999555 96.703888) (end 106.066872 96.715504) (width 0.12) (layer "F.Cu") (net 2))
 (arc (start 126.923509 99) (mid 127.347773 98.824264) (end 127.523509 98.4) (width 0.3) (layer "F.Cu") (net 2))
 (segment (start 141.242547 74.214476) (end 148.03983 67.613524) (width 0.3) (layer "B.Cu") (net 2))
 (segment (start 154.325461 61.25575) (end 154.325461 43.621699) (width 0.3) (layer "B.Cu") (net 2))
 (segment (start 154.325461 43.621699) (end 154.325461 33.285919) (width 0.3) (layer "B.Cu") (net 2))
 (segment (start 139.723509 91.15) (end 139.723509 89.53445) (width 0.3) (layer "B.Cu") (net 2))
 (segment (start 132.123509 97.65) (end 132.123509 92.65) (width 0.3) (layer "B.Cu") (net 2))
 (segment (start 139.723509 89.53445) (end 139.723509 87.49532) (width 0.3) (layer "B.Cu") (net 2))
 (segment (start 139.723509 91.645) (end 139.723509 91.15) (width 0.3) (layer "B.Cu") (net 2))
 (segment (start 132.723509 92.05) (end 139.318509 92.05) (width 0.3) (layer "B.Cu") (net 2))
 (segment (start 153.187761 62.614283) (end 154.143464 61.686184) (width 0.3) (layer "B.Cu") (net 2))
 (segment (start 148.03983 67.613524) (end 149.389174 66.303153) (width 0.3) (layer "B.Cu") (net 2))
 (segment (start 139.723509 87.49532) (end 139.723509 75.943333) (width 0.3) (layer "B.Cu") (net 2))
 (segment (start 149.389174 66.303153) (end 153.187761 62.614283) (width 0.3) (layer "B.Cu") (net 2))
 (segment (start 139.905506 75.512898) (end 141.242547 74.214476) (width 0.3) (layer "B.Cu") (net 2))
 (arc (start 139.723509 75.943333) (mid 139.770878 75.709668) (end 139.905506 75.512898) (width 0.3) (layer "B.Cu") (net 2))
 (arc (start 132.123509 92.65) (mid 132.299245 92.225735) (end 132.723509 92.05) (width 0.3) (layer "B.Cu") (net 2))
 (arc (start 154.143464 61.686184) (mid 154.278092 61.489415) (end 154.325461 61.25575) (width 0.3) (layer "B.Cu") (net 2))
 (arc (start 139.318509 92.05) (mid 139.604887 91.931378) (end 139.723509 91.645) (width 0.3) (layer "B.Cu") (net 2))
 (segment (start 130.797372 99.95) (end 226.632972 99.95) (width 0.12) (layer "F.Cu") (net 7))
 (segment (start 115.92 99.45) (end 128.649645 99.45) (width 0.12) (layer "F.Cu") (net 7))
 (segment (start 102.199999 97.05) (end 105.928451 97.05) (width 0.12) (layer "F.Cu") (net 7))
 (segment (start 106.069542 97.066824) (end 115.92 99.45) (width 0.12) (layer "F.Cu") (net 7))
 (segment (start 128.795167 99.467914) (end 130.651851 99.932085) (width 0.12) (layer "F.Cu") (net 7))
 (segment (start 227.026722 99.55625) (end 227.026722 99.075) (width 0.12) (layer "F.Cu") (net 7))
 (segment (start 101.6 98.8) (end 101.6 97.65) (width 0.12) (layer "F.Cu") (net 7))
 (arc (start 226.632972 99.95) (mid 226.911395 99.834673) (end 227.026722 99.55625) (width 0.12) (layer "F.Cu") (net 7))
 (arc (start 128.649645 99.45) (mid 128.722955 99.454495) (end 128.795167 99.467914) (width 0.12) (layer "F.Cu") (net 7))
 (arc (start 101.6 97.65) (mid 101.775735 97.225735) (end 102.199999 97.05) (width 0.12) (layer "F.Cu") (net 7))
 (arc (start 130.651851 99.932085) (mid 130.724062 99.945504) (end 130.797372 99.95) (width 0.12) (layer "F.Cu") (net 7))
 (arc (start 105.928451 97.05) (mid 105.999496 97.054221) (end 106.069542 97.066824) (width 0.12) (layer "F.Cu") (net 7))
 (segment (start 263.641403 101.2825) (end 263.656404 101.2675) (width 0.12) (layer "F.Cu") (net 4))
 (segment (start 102.199999 103.6) (end 105.918373 103.6) (width 0.12) (layer "F.Cu") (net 4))
 (segment (start 101.6 101.2) (end 101.6 103) (width 0.12) (layer "F.Cu") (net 4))
 (segment (start 128.795167 100.867914) (end 130.651851 101.332085) (width 0.12) (layer "F.Cu") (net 4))
 (segment (start 106.078659 103.578194) (end 115.92 100.85) (width 0.12) (layer "F.Cu") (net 4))
 (segment (start 115.92 100.85) (end 128.649645 100.85) (width 0.12) (layer "F.Cu") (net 4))
 (segment (start 130.797372 101.35) (end 263.478444 101.35) (width 0.12) (layer "F.Cu") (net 4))
 (segment (start 263.819363 101.2) (end 265.173904 101.2) (width 0.12) (layer "F.Cu") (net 4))
 (arc (start 263.656404 101.2675) (mid 263.73117 101.217542) (end 263.819363 101.2) (width 0.12) (layer "F.Cu") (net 4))
 (arc (start 105.918373 103.6) (mid 105.999254 103.594523) (end 106.078659 103.578194) (width 0.12) (layer "F.Cu") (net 4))
 (arc (start 101.6 103) (mid 101.775735 103.424264) (end 102.199999 103.6) (width 0.12) (layer "F.Cu") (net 4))
 (arc (start 130.651851 101.332085) (mid 130.724062 101.345504) (end 130.797372 101.35) (width 0.12) (layer "F.Cu") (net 4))
 (arc (start 128.649645 100.85) (mid 128.722955 100.854495) (end 128.795167 100.867914) (width 0.12) (layer "F.Cu") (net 4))
 (arc (start 263.478444 101.35) (mid 263.566637 101.332457) (end 263.641403 101.2825) (width 0.12) (layer "F.Cu") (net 4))
 (segment (start 106.069542 97.366824) (end 115.92 99.75) (width 0.12) (layer "F.Cu") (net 8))
 (segment (start 130.797372 100.25) (end 227.147972 100.25) (width 0.12) (layer "F.Cu") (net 8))
 (segment (start 115.92 99.75) (end 128.649645 99.75) (width 0.12) (layer "F.Cu") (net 8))
 (segment (start 128.795167 99.767914) (end 130.651851 100.232085) (width 0.12) (layer "F.Cu") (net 8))
 (segment (start 102 98.8) (end 102 97.95) (width 0.12) (layer "F.Cu") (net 8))
 (segment (start 227.676722 99.72125) (end 227.676722 99.075) (width 0.12) (layer "F.Cu") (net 8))
 (segment (start 102.6 97.35) (end 105.928451 97.35) (width 0.12) (layer "F.Cu") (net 8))
 (arc (start 105.928451 97.35) (mid 105.999496 97.354221) (end 106.069542 97.366824) (width 0.12) (layer "F.Cu") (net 8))
 (arc (start 130.651851 100.232085) (mid 130.724062 100.245504) (end 130.797372 100.25) (width 0.12) (layer "F.Cu") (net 8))
 (arc (start 102 97.95) (mid 102.175735 97.525735) (end 102.6 97.35) (width 0.12) (layer "F.Cu") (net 8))
 (arc (start 128.649645 99.75) (mid 128.722955 99.754495) (end 128.795167 99.767914) (width 0.12) (layer "F.Cu") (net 8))
 (arc (start 227.147972 100.25) (mid 227.521854 100.095132) (end 227.676722 99.72125) (width 0.12) (layer "F.Cu") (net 8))
 (segment (start 128.795167 100.517914) (end 130.651851 100.982085) (width 0.12) (layer "F.Cu") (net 3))
 (segment (start 115.92 100.5) (end 128.649645 100.5) (width 0.12) (layer "F.Cu") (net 3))
 (segment (start 264.422432 100.4) (end 265.173904 100.4) (width 0.12) (layer "F.Cu") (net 3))
 (segment (start 102.6 103.2) (end 105.919805 103.2) (width 0.12) (layer "F.Cu") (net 3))
 (segment (start 130.797372 101) (end 263.325375 101) (width 0.12) (layer "F.Cu") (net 3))
 (segment (start 102 101.2) (end 102 102.6) (width 0.12) (layer "F.Cu") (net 3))
 (segment (start 106.077379 103.178939) (end 115.92 100.5) (width 0.12) (layer "F.Cu") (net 3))
 (segment (start 263.749639 100.824264) (end 263.998168 100.575735) (width 0.12) (layer "F.Cu") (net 3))
 (arc (start 263.325375 101) (mid 263.554985 100.954327) (end 263.749639 100.824264) (width 0.12) (layer "F.Cu") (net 3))
 (arc (start 263.998168 100.575735) (mid 264.192822 100.445672) (end 264.422432 100.4) (width 0.12) (layer "F.Cu") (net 3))
 (arc (start 130.651851 100.982085) (mid 130.724062 100.995504) (end 130.797372 101) (width 0.12) (layer "F.Cu") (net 3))
 (arc (start 102 102.6) (mid 102.175735 103.024264) (end 102.6 103.2) (width 0.12) (layer "F.Cu") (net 3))
 (arc (start 128.649645 100.5) (mid 128.722955 100.504495) (end 128.795167 100.517914) (width 0.12) (layer "F.Cu") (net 3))
 (arc (start 105.919805 103.2) (mid 105.999293 103.194711) (end 106.077379 103.178939) (width 0.12) (layer "F.Cu") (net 3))
 (segment (start 102.4 98.8) (end 102.4 98.1675) (width 0.12) (layer "F.Cu") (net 9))
 (segment (start 228.326722 99.95) (end 228.326722 99.075) (width 0.12) (layer "F.Cu") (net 9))
 (segment (start 115.92 100.05) (end 128.649645 100.05) (width 0.12) (layer "F.Cu") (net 9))
 (segment (start 102.9175 97.65) (end 105.928451 97.65) (width 0.12) (layer "F.Cu") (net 9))
 (segment (start 130.797372 100.55) (end 227.726722 100.55) (width 0.12) (layer "F.Cu") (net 9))
 (segment (start 106.069542 97.666824) (end 115.92 100.05) (width 0.12) (layer "F.Cu") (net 9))
 (segment (start 128.795167 100.067914) (end 130.651851 100.532085) (width 0.12) (layer "F.Cu") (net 9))
 (segment (start 228.326722 99.075) (end 229.536722 99.08) (width 0.12) (layer "F.Cu") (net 9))
 (arc (start 130.651851 100.532085) (mid 130.724062 100.545504) (end 130.797372 100.55) (width 0.12) (layer "F.Cu") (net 9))
 (arc (start 102.4 98.1675) (mid 102.551572 97.801572) (end 102.9175 97.65) (width 0.12) (layer "F.Cu") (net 9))
 (arc (start 227.726722 100.55) (mid 228.150986 100.374264) (end 228.326722 99.95) (width 0.12) (layer "F.Cu") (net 9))
 (arc (start 128.649645 100.05) (mid 128.722955 100.054495) (end 128.795167 100.067914) (width 0.12) (layer "F.Cu") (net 9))
 (arc (start 105.928451 97.65) (mid 105.999496 97.654221) (end 106.069542 97.666824) (width 0.12) (layer "F.Cu") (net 9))
 (segment (start 266.936544 101.319587) (end 267.423904 102.25) (width 0.15) (layer "F.Cu") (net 5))
 (segment (start 103 102.6) (end 105.2 102.6) (width 0.15) (layer "F.Cu") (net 5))
 (segment (start 230.526722 96.92) (end 230.526722 96.05) (width 0.15) (layer "F.Cu") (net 5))
 (segment (start 227.026722 96.925) (end 227.026722 96.05) (width 0.15) (layer "F.Cu") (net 5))
 (segment (start 102.4 101.2) (end 102.4 102) (width 0.15) (layer "F.Cu") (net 5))
 (segment (start 266.573904 101.2) (end 266.738904 101.2) (width 0.15) (layer "F.Cu") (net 5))
 (segment (start 266.873904 101.2) (end 268.473904 101.28) (width 0.15) (layer "F.Cu") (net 5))
 (via (at 105.2 102.6) (size 0.6) (drill 0.3) (layers "F.Cu" "B.Cu") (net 5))
 (via (at 227.026722 96.05) (size 0.6) (drill 0.3) (layers "F.Cu" "B.Cu") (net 5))
 (via (at 230.526722 96.05) (size 0.6) (drill 0.3) (layers "F.Cu" "B.Cu") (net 5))
 (via (at 267.423904 102.25) (size 0.6) (drill 0.3) (layers "F.Cu" "B.Cu") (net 5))
 (arc (start 266.738904 101.2) (mid 266.854406 101.232223) (end 266.936544 101.319587) (width 0.15) (layer "F.Cu") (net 5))
 (arc (start 102.4 102) (mid 102.575735 102.424264) (end 103 102.6) (width 0.15) (layer "F.Cu") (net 5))
 (segment (start 227.026722 101.2) (end 227.026722 96.05) (width 0.15) (layer "B.Cu") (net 5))
 (segment (start 265.973803 101.298371) (end 267.423904 102.25) (width 0.15) (layer "B.Cu") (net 5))
 (segment (start 230.526722 101.2) (end 230.526722 96.05) (width 0.15) (layer "B.Cu") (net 5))
 (segment (start 105.2 102.6) (end 105.95787 102.6) (width 0.15) (layer "B.Cu") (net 5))
 (segment (start 106.041716 102.594112) (end 115.878283 101.205887) (width 0.15) (layer "B.Cu") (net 5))
 (segment (start 115.962129 101.2) (end 265.644609 101.2) (width 0.15) (layer "B.Cu") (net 5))
 (arc (start 105.95787 102.6) (mid 105.999896 102.598526) (end 106.041716 102.594112) (width 0.15) (layer "B.Cu") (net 5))
 (arc (start 115.878283 101.205887) (mid 115.920103 101.201473) (end 115.962129 101.2) (width 0.15) (layer "B.Cu") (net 5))
 (arc (start 265.644609 101.2) (mid 265.816397 101.225118) (end 265.973803 101.298371) (width 0.15) (layer "B.Cu") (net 5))
 (segment (start 224.996722 98.337499) (end 224.996722 96.4) (width 0.15) (layer "F.Cu") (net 6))
 (segment (start 228.326722 96.925) (end 229.566722 96.92) (width 0.15) (layer "F.Cu") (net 6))
 (segment (start 266.573904 100.4) (end 266.738904 100.4) (width 0.15) (layer "F.Cu") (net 6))
 (segment (start 266.936544 100.280412) (end 267.423904 99.35) (width 0.15) (layer "F.Cu") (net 6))
 (segment (start 102.8 101.2) (end 102.8 101.42) (width 0.15) (layer "F.Cu") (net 6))
 (segment (start 224.996722 96.4) (end 224.996722 95.7675) (width 0.15) (layer "F.Cu") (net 6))
 (segment (start 230.556722 99.08) (end 229.719798 97.613032) (width 0.15) (layer "F.Cu") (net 6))
 (segment (start 225.746722 98.675) (end 225.334222 98.675) (width 0.15) (layer "F.Cu") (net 6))
 (segment (start 230.556722 99.08) (end 231.206722 99.08) (width 0.15) (layer "F.Cu") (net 6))
 (segment (start 227.676722 95.85) (end 227.676722 96.6325) (width 0.15) (layer "F.Cu") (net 6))
 (segment (start 227.969222 96.925) (end 228.326722 96.925) (width 0.15) (layer "F.Cu") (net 6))
 (segment (start 102.960996 101.680498) (end 103.6 102) (width 0.15) (layer "F.Cu") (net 6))
 (segment (start 225.514222 95.25) (end 227.076722 95.25) (width 0.15) (layer "F.Cu") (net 6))
 (segment (start 229.649113 97.414348) (end 229.566722 96.92) (width 0.15) (layer "F.Cu") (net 6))
 (segment (start 266.873904 100.4) (end 268.473904 100.32) (width 0.15) (layer "F.Cu") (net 6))
 (via (at 267.423904 99.35) (size 0.6) (drill 0.3) (layers "F.Cu" "B.Cu") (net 6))
 (via (at 224.996722 96.4) (size 0.6) (drill 0.3) (layers "F.Cu" "B.Cu") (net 6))
 (via (at 231.206722 99.08) (size 0.6) (drill 0.3) (layers "F.Cu" "B.Cu") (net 6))
 (via (at 103.6 102) (size 0.6) (drill 0.3) (layers "F.Cu" "B.Cu") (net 6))
 (arc (start 227.676722 96.6325) (mid 227.762393 96.839328) (end 227.969222 96.925) (width 0.15) (layer "F.Cu") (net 6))
 (arc (start 225.334222 98.675) (mid 225.095573 98.576148) (end 224.996722 98.337499) (width 0.15) (layer "F.Cu") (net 6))
 (arc (start 227.076722 95.25) (mid 227.500986 95.425735) (end 227.676722 95.85) (width 0.15) (layer "F.Cu") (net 6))
 (arc (start 266.738904 100.4) (mid 266.854406 100.367776) (end 266.936544 100.280412) (width 0.15) (layer "F.Cu") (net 6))
 (arc (start 229.719798 97.613032) (mid 229.675658 97.51682) (end 229.649113 97.414348) (width 0.15) (layer "F.Cu") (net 6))
 (arc (start 224.996722 95.7675) (mid 225.148294 95.401572) (end 225.514222 95.25) (width 0.15) (layer "F.Cu") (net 6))
 (arc (start 102.8 101.42) (mid 102.843497 101.573117) (end 102.960996 101.680498) (width 0.15) (layer "F.Cu") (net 6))
 (segment (start 103.6 102) (end 105.95787 102) (width 0.15) (layer "B.Cu") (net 6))
 (segment (start 232.214933 100.6) (end 265.617314 100.6) (width 0.15) (layer "B.Cu") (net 6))
 (segment (start 265.986701 100.472814) (end 267.423904 99.35) (width 0.15) (layer "B.Cu") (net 6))
 (segment (start 224.996722 100) (end 224.996722 96.4) (width 0.15) (layer "B.Cu") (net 6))
 (segment (start 231.206722 99.08) (end 231.65684 100.220299) (width 0.15) (layer "B.Cu") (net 6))
 (segment (start 115.962129 100.6) (end 224.396722 100.6) (width 0.15) (layer "B.Cu") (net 6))
 (segment (start 106.041716 101.994112) (end 115.878283 100.605887) (width 0.15) (layer "B.Cu") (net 6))
 (arc (start 105.95787 102) (mid 105.999896 101.998526) (end 106.041716 101.994112) (width 0.15) (layer "B.Cu") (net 6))
 (arc (start 115.878283 100.605887) (mid 115.920103 100.601473) (end 115.962129 100.6) (width 0.15) (layer "B.Cu") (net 6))
 (arc (start 231.65684 100.220299) (mid 231.877427 100.496074) (end 232.214933 100.6) (width 0.15) (layer "B.Cu") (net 6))
 (arc (start 265.617314 100.6) (mid 265.812649 100.567313) (end 265.986701 100.472814) (width 0.15) (layer "B.Cu") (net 6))
 (arc (start 224.396722 100.6) (mid 224.820986 100.424264) (end 224.996722 100) (width 0.15) (layer "B.Cu") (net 6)))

